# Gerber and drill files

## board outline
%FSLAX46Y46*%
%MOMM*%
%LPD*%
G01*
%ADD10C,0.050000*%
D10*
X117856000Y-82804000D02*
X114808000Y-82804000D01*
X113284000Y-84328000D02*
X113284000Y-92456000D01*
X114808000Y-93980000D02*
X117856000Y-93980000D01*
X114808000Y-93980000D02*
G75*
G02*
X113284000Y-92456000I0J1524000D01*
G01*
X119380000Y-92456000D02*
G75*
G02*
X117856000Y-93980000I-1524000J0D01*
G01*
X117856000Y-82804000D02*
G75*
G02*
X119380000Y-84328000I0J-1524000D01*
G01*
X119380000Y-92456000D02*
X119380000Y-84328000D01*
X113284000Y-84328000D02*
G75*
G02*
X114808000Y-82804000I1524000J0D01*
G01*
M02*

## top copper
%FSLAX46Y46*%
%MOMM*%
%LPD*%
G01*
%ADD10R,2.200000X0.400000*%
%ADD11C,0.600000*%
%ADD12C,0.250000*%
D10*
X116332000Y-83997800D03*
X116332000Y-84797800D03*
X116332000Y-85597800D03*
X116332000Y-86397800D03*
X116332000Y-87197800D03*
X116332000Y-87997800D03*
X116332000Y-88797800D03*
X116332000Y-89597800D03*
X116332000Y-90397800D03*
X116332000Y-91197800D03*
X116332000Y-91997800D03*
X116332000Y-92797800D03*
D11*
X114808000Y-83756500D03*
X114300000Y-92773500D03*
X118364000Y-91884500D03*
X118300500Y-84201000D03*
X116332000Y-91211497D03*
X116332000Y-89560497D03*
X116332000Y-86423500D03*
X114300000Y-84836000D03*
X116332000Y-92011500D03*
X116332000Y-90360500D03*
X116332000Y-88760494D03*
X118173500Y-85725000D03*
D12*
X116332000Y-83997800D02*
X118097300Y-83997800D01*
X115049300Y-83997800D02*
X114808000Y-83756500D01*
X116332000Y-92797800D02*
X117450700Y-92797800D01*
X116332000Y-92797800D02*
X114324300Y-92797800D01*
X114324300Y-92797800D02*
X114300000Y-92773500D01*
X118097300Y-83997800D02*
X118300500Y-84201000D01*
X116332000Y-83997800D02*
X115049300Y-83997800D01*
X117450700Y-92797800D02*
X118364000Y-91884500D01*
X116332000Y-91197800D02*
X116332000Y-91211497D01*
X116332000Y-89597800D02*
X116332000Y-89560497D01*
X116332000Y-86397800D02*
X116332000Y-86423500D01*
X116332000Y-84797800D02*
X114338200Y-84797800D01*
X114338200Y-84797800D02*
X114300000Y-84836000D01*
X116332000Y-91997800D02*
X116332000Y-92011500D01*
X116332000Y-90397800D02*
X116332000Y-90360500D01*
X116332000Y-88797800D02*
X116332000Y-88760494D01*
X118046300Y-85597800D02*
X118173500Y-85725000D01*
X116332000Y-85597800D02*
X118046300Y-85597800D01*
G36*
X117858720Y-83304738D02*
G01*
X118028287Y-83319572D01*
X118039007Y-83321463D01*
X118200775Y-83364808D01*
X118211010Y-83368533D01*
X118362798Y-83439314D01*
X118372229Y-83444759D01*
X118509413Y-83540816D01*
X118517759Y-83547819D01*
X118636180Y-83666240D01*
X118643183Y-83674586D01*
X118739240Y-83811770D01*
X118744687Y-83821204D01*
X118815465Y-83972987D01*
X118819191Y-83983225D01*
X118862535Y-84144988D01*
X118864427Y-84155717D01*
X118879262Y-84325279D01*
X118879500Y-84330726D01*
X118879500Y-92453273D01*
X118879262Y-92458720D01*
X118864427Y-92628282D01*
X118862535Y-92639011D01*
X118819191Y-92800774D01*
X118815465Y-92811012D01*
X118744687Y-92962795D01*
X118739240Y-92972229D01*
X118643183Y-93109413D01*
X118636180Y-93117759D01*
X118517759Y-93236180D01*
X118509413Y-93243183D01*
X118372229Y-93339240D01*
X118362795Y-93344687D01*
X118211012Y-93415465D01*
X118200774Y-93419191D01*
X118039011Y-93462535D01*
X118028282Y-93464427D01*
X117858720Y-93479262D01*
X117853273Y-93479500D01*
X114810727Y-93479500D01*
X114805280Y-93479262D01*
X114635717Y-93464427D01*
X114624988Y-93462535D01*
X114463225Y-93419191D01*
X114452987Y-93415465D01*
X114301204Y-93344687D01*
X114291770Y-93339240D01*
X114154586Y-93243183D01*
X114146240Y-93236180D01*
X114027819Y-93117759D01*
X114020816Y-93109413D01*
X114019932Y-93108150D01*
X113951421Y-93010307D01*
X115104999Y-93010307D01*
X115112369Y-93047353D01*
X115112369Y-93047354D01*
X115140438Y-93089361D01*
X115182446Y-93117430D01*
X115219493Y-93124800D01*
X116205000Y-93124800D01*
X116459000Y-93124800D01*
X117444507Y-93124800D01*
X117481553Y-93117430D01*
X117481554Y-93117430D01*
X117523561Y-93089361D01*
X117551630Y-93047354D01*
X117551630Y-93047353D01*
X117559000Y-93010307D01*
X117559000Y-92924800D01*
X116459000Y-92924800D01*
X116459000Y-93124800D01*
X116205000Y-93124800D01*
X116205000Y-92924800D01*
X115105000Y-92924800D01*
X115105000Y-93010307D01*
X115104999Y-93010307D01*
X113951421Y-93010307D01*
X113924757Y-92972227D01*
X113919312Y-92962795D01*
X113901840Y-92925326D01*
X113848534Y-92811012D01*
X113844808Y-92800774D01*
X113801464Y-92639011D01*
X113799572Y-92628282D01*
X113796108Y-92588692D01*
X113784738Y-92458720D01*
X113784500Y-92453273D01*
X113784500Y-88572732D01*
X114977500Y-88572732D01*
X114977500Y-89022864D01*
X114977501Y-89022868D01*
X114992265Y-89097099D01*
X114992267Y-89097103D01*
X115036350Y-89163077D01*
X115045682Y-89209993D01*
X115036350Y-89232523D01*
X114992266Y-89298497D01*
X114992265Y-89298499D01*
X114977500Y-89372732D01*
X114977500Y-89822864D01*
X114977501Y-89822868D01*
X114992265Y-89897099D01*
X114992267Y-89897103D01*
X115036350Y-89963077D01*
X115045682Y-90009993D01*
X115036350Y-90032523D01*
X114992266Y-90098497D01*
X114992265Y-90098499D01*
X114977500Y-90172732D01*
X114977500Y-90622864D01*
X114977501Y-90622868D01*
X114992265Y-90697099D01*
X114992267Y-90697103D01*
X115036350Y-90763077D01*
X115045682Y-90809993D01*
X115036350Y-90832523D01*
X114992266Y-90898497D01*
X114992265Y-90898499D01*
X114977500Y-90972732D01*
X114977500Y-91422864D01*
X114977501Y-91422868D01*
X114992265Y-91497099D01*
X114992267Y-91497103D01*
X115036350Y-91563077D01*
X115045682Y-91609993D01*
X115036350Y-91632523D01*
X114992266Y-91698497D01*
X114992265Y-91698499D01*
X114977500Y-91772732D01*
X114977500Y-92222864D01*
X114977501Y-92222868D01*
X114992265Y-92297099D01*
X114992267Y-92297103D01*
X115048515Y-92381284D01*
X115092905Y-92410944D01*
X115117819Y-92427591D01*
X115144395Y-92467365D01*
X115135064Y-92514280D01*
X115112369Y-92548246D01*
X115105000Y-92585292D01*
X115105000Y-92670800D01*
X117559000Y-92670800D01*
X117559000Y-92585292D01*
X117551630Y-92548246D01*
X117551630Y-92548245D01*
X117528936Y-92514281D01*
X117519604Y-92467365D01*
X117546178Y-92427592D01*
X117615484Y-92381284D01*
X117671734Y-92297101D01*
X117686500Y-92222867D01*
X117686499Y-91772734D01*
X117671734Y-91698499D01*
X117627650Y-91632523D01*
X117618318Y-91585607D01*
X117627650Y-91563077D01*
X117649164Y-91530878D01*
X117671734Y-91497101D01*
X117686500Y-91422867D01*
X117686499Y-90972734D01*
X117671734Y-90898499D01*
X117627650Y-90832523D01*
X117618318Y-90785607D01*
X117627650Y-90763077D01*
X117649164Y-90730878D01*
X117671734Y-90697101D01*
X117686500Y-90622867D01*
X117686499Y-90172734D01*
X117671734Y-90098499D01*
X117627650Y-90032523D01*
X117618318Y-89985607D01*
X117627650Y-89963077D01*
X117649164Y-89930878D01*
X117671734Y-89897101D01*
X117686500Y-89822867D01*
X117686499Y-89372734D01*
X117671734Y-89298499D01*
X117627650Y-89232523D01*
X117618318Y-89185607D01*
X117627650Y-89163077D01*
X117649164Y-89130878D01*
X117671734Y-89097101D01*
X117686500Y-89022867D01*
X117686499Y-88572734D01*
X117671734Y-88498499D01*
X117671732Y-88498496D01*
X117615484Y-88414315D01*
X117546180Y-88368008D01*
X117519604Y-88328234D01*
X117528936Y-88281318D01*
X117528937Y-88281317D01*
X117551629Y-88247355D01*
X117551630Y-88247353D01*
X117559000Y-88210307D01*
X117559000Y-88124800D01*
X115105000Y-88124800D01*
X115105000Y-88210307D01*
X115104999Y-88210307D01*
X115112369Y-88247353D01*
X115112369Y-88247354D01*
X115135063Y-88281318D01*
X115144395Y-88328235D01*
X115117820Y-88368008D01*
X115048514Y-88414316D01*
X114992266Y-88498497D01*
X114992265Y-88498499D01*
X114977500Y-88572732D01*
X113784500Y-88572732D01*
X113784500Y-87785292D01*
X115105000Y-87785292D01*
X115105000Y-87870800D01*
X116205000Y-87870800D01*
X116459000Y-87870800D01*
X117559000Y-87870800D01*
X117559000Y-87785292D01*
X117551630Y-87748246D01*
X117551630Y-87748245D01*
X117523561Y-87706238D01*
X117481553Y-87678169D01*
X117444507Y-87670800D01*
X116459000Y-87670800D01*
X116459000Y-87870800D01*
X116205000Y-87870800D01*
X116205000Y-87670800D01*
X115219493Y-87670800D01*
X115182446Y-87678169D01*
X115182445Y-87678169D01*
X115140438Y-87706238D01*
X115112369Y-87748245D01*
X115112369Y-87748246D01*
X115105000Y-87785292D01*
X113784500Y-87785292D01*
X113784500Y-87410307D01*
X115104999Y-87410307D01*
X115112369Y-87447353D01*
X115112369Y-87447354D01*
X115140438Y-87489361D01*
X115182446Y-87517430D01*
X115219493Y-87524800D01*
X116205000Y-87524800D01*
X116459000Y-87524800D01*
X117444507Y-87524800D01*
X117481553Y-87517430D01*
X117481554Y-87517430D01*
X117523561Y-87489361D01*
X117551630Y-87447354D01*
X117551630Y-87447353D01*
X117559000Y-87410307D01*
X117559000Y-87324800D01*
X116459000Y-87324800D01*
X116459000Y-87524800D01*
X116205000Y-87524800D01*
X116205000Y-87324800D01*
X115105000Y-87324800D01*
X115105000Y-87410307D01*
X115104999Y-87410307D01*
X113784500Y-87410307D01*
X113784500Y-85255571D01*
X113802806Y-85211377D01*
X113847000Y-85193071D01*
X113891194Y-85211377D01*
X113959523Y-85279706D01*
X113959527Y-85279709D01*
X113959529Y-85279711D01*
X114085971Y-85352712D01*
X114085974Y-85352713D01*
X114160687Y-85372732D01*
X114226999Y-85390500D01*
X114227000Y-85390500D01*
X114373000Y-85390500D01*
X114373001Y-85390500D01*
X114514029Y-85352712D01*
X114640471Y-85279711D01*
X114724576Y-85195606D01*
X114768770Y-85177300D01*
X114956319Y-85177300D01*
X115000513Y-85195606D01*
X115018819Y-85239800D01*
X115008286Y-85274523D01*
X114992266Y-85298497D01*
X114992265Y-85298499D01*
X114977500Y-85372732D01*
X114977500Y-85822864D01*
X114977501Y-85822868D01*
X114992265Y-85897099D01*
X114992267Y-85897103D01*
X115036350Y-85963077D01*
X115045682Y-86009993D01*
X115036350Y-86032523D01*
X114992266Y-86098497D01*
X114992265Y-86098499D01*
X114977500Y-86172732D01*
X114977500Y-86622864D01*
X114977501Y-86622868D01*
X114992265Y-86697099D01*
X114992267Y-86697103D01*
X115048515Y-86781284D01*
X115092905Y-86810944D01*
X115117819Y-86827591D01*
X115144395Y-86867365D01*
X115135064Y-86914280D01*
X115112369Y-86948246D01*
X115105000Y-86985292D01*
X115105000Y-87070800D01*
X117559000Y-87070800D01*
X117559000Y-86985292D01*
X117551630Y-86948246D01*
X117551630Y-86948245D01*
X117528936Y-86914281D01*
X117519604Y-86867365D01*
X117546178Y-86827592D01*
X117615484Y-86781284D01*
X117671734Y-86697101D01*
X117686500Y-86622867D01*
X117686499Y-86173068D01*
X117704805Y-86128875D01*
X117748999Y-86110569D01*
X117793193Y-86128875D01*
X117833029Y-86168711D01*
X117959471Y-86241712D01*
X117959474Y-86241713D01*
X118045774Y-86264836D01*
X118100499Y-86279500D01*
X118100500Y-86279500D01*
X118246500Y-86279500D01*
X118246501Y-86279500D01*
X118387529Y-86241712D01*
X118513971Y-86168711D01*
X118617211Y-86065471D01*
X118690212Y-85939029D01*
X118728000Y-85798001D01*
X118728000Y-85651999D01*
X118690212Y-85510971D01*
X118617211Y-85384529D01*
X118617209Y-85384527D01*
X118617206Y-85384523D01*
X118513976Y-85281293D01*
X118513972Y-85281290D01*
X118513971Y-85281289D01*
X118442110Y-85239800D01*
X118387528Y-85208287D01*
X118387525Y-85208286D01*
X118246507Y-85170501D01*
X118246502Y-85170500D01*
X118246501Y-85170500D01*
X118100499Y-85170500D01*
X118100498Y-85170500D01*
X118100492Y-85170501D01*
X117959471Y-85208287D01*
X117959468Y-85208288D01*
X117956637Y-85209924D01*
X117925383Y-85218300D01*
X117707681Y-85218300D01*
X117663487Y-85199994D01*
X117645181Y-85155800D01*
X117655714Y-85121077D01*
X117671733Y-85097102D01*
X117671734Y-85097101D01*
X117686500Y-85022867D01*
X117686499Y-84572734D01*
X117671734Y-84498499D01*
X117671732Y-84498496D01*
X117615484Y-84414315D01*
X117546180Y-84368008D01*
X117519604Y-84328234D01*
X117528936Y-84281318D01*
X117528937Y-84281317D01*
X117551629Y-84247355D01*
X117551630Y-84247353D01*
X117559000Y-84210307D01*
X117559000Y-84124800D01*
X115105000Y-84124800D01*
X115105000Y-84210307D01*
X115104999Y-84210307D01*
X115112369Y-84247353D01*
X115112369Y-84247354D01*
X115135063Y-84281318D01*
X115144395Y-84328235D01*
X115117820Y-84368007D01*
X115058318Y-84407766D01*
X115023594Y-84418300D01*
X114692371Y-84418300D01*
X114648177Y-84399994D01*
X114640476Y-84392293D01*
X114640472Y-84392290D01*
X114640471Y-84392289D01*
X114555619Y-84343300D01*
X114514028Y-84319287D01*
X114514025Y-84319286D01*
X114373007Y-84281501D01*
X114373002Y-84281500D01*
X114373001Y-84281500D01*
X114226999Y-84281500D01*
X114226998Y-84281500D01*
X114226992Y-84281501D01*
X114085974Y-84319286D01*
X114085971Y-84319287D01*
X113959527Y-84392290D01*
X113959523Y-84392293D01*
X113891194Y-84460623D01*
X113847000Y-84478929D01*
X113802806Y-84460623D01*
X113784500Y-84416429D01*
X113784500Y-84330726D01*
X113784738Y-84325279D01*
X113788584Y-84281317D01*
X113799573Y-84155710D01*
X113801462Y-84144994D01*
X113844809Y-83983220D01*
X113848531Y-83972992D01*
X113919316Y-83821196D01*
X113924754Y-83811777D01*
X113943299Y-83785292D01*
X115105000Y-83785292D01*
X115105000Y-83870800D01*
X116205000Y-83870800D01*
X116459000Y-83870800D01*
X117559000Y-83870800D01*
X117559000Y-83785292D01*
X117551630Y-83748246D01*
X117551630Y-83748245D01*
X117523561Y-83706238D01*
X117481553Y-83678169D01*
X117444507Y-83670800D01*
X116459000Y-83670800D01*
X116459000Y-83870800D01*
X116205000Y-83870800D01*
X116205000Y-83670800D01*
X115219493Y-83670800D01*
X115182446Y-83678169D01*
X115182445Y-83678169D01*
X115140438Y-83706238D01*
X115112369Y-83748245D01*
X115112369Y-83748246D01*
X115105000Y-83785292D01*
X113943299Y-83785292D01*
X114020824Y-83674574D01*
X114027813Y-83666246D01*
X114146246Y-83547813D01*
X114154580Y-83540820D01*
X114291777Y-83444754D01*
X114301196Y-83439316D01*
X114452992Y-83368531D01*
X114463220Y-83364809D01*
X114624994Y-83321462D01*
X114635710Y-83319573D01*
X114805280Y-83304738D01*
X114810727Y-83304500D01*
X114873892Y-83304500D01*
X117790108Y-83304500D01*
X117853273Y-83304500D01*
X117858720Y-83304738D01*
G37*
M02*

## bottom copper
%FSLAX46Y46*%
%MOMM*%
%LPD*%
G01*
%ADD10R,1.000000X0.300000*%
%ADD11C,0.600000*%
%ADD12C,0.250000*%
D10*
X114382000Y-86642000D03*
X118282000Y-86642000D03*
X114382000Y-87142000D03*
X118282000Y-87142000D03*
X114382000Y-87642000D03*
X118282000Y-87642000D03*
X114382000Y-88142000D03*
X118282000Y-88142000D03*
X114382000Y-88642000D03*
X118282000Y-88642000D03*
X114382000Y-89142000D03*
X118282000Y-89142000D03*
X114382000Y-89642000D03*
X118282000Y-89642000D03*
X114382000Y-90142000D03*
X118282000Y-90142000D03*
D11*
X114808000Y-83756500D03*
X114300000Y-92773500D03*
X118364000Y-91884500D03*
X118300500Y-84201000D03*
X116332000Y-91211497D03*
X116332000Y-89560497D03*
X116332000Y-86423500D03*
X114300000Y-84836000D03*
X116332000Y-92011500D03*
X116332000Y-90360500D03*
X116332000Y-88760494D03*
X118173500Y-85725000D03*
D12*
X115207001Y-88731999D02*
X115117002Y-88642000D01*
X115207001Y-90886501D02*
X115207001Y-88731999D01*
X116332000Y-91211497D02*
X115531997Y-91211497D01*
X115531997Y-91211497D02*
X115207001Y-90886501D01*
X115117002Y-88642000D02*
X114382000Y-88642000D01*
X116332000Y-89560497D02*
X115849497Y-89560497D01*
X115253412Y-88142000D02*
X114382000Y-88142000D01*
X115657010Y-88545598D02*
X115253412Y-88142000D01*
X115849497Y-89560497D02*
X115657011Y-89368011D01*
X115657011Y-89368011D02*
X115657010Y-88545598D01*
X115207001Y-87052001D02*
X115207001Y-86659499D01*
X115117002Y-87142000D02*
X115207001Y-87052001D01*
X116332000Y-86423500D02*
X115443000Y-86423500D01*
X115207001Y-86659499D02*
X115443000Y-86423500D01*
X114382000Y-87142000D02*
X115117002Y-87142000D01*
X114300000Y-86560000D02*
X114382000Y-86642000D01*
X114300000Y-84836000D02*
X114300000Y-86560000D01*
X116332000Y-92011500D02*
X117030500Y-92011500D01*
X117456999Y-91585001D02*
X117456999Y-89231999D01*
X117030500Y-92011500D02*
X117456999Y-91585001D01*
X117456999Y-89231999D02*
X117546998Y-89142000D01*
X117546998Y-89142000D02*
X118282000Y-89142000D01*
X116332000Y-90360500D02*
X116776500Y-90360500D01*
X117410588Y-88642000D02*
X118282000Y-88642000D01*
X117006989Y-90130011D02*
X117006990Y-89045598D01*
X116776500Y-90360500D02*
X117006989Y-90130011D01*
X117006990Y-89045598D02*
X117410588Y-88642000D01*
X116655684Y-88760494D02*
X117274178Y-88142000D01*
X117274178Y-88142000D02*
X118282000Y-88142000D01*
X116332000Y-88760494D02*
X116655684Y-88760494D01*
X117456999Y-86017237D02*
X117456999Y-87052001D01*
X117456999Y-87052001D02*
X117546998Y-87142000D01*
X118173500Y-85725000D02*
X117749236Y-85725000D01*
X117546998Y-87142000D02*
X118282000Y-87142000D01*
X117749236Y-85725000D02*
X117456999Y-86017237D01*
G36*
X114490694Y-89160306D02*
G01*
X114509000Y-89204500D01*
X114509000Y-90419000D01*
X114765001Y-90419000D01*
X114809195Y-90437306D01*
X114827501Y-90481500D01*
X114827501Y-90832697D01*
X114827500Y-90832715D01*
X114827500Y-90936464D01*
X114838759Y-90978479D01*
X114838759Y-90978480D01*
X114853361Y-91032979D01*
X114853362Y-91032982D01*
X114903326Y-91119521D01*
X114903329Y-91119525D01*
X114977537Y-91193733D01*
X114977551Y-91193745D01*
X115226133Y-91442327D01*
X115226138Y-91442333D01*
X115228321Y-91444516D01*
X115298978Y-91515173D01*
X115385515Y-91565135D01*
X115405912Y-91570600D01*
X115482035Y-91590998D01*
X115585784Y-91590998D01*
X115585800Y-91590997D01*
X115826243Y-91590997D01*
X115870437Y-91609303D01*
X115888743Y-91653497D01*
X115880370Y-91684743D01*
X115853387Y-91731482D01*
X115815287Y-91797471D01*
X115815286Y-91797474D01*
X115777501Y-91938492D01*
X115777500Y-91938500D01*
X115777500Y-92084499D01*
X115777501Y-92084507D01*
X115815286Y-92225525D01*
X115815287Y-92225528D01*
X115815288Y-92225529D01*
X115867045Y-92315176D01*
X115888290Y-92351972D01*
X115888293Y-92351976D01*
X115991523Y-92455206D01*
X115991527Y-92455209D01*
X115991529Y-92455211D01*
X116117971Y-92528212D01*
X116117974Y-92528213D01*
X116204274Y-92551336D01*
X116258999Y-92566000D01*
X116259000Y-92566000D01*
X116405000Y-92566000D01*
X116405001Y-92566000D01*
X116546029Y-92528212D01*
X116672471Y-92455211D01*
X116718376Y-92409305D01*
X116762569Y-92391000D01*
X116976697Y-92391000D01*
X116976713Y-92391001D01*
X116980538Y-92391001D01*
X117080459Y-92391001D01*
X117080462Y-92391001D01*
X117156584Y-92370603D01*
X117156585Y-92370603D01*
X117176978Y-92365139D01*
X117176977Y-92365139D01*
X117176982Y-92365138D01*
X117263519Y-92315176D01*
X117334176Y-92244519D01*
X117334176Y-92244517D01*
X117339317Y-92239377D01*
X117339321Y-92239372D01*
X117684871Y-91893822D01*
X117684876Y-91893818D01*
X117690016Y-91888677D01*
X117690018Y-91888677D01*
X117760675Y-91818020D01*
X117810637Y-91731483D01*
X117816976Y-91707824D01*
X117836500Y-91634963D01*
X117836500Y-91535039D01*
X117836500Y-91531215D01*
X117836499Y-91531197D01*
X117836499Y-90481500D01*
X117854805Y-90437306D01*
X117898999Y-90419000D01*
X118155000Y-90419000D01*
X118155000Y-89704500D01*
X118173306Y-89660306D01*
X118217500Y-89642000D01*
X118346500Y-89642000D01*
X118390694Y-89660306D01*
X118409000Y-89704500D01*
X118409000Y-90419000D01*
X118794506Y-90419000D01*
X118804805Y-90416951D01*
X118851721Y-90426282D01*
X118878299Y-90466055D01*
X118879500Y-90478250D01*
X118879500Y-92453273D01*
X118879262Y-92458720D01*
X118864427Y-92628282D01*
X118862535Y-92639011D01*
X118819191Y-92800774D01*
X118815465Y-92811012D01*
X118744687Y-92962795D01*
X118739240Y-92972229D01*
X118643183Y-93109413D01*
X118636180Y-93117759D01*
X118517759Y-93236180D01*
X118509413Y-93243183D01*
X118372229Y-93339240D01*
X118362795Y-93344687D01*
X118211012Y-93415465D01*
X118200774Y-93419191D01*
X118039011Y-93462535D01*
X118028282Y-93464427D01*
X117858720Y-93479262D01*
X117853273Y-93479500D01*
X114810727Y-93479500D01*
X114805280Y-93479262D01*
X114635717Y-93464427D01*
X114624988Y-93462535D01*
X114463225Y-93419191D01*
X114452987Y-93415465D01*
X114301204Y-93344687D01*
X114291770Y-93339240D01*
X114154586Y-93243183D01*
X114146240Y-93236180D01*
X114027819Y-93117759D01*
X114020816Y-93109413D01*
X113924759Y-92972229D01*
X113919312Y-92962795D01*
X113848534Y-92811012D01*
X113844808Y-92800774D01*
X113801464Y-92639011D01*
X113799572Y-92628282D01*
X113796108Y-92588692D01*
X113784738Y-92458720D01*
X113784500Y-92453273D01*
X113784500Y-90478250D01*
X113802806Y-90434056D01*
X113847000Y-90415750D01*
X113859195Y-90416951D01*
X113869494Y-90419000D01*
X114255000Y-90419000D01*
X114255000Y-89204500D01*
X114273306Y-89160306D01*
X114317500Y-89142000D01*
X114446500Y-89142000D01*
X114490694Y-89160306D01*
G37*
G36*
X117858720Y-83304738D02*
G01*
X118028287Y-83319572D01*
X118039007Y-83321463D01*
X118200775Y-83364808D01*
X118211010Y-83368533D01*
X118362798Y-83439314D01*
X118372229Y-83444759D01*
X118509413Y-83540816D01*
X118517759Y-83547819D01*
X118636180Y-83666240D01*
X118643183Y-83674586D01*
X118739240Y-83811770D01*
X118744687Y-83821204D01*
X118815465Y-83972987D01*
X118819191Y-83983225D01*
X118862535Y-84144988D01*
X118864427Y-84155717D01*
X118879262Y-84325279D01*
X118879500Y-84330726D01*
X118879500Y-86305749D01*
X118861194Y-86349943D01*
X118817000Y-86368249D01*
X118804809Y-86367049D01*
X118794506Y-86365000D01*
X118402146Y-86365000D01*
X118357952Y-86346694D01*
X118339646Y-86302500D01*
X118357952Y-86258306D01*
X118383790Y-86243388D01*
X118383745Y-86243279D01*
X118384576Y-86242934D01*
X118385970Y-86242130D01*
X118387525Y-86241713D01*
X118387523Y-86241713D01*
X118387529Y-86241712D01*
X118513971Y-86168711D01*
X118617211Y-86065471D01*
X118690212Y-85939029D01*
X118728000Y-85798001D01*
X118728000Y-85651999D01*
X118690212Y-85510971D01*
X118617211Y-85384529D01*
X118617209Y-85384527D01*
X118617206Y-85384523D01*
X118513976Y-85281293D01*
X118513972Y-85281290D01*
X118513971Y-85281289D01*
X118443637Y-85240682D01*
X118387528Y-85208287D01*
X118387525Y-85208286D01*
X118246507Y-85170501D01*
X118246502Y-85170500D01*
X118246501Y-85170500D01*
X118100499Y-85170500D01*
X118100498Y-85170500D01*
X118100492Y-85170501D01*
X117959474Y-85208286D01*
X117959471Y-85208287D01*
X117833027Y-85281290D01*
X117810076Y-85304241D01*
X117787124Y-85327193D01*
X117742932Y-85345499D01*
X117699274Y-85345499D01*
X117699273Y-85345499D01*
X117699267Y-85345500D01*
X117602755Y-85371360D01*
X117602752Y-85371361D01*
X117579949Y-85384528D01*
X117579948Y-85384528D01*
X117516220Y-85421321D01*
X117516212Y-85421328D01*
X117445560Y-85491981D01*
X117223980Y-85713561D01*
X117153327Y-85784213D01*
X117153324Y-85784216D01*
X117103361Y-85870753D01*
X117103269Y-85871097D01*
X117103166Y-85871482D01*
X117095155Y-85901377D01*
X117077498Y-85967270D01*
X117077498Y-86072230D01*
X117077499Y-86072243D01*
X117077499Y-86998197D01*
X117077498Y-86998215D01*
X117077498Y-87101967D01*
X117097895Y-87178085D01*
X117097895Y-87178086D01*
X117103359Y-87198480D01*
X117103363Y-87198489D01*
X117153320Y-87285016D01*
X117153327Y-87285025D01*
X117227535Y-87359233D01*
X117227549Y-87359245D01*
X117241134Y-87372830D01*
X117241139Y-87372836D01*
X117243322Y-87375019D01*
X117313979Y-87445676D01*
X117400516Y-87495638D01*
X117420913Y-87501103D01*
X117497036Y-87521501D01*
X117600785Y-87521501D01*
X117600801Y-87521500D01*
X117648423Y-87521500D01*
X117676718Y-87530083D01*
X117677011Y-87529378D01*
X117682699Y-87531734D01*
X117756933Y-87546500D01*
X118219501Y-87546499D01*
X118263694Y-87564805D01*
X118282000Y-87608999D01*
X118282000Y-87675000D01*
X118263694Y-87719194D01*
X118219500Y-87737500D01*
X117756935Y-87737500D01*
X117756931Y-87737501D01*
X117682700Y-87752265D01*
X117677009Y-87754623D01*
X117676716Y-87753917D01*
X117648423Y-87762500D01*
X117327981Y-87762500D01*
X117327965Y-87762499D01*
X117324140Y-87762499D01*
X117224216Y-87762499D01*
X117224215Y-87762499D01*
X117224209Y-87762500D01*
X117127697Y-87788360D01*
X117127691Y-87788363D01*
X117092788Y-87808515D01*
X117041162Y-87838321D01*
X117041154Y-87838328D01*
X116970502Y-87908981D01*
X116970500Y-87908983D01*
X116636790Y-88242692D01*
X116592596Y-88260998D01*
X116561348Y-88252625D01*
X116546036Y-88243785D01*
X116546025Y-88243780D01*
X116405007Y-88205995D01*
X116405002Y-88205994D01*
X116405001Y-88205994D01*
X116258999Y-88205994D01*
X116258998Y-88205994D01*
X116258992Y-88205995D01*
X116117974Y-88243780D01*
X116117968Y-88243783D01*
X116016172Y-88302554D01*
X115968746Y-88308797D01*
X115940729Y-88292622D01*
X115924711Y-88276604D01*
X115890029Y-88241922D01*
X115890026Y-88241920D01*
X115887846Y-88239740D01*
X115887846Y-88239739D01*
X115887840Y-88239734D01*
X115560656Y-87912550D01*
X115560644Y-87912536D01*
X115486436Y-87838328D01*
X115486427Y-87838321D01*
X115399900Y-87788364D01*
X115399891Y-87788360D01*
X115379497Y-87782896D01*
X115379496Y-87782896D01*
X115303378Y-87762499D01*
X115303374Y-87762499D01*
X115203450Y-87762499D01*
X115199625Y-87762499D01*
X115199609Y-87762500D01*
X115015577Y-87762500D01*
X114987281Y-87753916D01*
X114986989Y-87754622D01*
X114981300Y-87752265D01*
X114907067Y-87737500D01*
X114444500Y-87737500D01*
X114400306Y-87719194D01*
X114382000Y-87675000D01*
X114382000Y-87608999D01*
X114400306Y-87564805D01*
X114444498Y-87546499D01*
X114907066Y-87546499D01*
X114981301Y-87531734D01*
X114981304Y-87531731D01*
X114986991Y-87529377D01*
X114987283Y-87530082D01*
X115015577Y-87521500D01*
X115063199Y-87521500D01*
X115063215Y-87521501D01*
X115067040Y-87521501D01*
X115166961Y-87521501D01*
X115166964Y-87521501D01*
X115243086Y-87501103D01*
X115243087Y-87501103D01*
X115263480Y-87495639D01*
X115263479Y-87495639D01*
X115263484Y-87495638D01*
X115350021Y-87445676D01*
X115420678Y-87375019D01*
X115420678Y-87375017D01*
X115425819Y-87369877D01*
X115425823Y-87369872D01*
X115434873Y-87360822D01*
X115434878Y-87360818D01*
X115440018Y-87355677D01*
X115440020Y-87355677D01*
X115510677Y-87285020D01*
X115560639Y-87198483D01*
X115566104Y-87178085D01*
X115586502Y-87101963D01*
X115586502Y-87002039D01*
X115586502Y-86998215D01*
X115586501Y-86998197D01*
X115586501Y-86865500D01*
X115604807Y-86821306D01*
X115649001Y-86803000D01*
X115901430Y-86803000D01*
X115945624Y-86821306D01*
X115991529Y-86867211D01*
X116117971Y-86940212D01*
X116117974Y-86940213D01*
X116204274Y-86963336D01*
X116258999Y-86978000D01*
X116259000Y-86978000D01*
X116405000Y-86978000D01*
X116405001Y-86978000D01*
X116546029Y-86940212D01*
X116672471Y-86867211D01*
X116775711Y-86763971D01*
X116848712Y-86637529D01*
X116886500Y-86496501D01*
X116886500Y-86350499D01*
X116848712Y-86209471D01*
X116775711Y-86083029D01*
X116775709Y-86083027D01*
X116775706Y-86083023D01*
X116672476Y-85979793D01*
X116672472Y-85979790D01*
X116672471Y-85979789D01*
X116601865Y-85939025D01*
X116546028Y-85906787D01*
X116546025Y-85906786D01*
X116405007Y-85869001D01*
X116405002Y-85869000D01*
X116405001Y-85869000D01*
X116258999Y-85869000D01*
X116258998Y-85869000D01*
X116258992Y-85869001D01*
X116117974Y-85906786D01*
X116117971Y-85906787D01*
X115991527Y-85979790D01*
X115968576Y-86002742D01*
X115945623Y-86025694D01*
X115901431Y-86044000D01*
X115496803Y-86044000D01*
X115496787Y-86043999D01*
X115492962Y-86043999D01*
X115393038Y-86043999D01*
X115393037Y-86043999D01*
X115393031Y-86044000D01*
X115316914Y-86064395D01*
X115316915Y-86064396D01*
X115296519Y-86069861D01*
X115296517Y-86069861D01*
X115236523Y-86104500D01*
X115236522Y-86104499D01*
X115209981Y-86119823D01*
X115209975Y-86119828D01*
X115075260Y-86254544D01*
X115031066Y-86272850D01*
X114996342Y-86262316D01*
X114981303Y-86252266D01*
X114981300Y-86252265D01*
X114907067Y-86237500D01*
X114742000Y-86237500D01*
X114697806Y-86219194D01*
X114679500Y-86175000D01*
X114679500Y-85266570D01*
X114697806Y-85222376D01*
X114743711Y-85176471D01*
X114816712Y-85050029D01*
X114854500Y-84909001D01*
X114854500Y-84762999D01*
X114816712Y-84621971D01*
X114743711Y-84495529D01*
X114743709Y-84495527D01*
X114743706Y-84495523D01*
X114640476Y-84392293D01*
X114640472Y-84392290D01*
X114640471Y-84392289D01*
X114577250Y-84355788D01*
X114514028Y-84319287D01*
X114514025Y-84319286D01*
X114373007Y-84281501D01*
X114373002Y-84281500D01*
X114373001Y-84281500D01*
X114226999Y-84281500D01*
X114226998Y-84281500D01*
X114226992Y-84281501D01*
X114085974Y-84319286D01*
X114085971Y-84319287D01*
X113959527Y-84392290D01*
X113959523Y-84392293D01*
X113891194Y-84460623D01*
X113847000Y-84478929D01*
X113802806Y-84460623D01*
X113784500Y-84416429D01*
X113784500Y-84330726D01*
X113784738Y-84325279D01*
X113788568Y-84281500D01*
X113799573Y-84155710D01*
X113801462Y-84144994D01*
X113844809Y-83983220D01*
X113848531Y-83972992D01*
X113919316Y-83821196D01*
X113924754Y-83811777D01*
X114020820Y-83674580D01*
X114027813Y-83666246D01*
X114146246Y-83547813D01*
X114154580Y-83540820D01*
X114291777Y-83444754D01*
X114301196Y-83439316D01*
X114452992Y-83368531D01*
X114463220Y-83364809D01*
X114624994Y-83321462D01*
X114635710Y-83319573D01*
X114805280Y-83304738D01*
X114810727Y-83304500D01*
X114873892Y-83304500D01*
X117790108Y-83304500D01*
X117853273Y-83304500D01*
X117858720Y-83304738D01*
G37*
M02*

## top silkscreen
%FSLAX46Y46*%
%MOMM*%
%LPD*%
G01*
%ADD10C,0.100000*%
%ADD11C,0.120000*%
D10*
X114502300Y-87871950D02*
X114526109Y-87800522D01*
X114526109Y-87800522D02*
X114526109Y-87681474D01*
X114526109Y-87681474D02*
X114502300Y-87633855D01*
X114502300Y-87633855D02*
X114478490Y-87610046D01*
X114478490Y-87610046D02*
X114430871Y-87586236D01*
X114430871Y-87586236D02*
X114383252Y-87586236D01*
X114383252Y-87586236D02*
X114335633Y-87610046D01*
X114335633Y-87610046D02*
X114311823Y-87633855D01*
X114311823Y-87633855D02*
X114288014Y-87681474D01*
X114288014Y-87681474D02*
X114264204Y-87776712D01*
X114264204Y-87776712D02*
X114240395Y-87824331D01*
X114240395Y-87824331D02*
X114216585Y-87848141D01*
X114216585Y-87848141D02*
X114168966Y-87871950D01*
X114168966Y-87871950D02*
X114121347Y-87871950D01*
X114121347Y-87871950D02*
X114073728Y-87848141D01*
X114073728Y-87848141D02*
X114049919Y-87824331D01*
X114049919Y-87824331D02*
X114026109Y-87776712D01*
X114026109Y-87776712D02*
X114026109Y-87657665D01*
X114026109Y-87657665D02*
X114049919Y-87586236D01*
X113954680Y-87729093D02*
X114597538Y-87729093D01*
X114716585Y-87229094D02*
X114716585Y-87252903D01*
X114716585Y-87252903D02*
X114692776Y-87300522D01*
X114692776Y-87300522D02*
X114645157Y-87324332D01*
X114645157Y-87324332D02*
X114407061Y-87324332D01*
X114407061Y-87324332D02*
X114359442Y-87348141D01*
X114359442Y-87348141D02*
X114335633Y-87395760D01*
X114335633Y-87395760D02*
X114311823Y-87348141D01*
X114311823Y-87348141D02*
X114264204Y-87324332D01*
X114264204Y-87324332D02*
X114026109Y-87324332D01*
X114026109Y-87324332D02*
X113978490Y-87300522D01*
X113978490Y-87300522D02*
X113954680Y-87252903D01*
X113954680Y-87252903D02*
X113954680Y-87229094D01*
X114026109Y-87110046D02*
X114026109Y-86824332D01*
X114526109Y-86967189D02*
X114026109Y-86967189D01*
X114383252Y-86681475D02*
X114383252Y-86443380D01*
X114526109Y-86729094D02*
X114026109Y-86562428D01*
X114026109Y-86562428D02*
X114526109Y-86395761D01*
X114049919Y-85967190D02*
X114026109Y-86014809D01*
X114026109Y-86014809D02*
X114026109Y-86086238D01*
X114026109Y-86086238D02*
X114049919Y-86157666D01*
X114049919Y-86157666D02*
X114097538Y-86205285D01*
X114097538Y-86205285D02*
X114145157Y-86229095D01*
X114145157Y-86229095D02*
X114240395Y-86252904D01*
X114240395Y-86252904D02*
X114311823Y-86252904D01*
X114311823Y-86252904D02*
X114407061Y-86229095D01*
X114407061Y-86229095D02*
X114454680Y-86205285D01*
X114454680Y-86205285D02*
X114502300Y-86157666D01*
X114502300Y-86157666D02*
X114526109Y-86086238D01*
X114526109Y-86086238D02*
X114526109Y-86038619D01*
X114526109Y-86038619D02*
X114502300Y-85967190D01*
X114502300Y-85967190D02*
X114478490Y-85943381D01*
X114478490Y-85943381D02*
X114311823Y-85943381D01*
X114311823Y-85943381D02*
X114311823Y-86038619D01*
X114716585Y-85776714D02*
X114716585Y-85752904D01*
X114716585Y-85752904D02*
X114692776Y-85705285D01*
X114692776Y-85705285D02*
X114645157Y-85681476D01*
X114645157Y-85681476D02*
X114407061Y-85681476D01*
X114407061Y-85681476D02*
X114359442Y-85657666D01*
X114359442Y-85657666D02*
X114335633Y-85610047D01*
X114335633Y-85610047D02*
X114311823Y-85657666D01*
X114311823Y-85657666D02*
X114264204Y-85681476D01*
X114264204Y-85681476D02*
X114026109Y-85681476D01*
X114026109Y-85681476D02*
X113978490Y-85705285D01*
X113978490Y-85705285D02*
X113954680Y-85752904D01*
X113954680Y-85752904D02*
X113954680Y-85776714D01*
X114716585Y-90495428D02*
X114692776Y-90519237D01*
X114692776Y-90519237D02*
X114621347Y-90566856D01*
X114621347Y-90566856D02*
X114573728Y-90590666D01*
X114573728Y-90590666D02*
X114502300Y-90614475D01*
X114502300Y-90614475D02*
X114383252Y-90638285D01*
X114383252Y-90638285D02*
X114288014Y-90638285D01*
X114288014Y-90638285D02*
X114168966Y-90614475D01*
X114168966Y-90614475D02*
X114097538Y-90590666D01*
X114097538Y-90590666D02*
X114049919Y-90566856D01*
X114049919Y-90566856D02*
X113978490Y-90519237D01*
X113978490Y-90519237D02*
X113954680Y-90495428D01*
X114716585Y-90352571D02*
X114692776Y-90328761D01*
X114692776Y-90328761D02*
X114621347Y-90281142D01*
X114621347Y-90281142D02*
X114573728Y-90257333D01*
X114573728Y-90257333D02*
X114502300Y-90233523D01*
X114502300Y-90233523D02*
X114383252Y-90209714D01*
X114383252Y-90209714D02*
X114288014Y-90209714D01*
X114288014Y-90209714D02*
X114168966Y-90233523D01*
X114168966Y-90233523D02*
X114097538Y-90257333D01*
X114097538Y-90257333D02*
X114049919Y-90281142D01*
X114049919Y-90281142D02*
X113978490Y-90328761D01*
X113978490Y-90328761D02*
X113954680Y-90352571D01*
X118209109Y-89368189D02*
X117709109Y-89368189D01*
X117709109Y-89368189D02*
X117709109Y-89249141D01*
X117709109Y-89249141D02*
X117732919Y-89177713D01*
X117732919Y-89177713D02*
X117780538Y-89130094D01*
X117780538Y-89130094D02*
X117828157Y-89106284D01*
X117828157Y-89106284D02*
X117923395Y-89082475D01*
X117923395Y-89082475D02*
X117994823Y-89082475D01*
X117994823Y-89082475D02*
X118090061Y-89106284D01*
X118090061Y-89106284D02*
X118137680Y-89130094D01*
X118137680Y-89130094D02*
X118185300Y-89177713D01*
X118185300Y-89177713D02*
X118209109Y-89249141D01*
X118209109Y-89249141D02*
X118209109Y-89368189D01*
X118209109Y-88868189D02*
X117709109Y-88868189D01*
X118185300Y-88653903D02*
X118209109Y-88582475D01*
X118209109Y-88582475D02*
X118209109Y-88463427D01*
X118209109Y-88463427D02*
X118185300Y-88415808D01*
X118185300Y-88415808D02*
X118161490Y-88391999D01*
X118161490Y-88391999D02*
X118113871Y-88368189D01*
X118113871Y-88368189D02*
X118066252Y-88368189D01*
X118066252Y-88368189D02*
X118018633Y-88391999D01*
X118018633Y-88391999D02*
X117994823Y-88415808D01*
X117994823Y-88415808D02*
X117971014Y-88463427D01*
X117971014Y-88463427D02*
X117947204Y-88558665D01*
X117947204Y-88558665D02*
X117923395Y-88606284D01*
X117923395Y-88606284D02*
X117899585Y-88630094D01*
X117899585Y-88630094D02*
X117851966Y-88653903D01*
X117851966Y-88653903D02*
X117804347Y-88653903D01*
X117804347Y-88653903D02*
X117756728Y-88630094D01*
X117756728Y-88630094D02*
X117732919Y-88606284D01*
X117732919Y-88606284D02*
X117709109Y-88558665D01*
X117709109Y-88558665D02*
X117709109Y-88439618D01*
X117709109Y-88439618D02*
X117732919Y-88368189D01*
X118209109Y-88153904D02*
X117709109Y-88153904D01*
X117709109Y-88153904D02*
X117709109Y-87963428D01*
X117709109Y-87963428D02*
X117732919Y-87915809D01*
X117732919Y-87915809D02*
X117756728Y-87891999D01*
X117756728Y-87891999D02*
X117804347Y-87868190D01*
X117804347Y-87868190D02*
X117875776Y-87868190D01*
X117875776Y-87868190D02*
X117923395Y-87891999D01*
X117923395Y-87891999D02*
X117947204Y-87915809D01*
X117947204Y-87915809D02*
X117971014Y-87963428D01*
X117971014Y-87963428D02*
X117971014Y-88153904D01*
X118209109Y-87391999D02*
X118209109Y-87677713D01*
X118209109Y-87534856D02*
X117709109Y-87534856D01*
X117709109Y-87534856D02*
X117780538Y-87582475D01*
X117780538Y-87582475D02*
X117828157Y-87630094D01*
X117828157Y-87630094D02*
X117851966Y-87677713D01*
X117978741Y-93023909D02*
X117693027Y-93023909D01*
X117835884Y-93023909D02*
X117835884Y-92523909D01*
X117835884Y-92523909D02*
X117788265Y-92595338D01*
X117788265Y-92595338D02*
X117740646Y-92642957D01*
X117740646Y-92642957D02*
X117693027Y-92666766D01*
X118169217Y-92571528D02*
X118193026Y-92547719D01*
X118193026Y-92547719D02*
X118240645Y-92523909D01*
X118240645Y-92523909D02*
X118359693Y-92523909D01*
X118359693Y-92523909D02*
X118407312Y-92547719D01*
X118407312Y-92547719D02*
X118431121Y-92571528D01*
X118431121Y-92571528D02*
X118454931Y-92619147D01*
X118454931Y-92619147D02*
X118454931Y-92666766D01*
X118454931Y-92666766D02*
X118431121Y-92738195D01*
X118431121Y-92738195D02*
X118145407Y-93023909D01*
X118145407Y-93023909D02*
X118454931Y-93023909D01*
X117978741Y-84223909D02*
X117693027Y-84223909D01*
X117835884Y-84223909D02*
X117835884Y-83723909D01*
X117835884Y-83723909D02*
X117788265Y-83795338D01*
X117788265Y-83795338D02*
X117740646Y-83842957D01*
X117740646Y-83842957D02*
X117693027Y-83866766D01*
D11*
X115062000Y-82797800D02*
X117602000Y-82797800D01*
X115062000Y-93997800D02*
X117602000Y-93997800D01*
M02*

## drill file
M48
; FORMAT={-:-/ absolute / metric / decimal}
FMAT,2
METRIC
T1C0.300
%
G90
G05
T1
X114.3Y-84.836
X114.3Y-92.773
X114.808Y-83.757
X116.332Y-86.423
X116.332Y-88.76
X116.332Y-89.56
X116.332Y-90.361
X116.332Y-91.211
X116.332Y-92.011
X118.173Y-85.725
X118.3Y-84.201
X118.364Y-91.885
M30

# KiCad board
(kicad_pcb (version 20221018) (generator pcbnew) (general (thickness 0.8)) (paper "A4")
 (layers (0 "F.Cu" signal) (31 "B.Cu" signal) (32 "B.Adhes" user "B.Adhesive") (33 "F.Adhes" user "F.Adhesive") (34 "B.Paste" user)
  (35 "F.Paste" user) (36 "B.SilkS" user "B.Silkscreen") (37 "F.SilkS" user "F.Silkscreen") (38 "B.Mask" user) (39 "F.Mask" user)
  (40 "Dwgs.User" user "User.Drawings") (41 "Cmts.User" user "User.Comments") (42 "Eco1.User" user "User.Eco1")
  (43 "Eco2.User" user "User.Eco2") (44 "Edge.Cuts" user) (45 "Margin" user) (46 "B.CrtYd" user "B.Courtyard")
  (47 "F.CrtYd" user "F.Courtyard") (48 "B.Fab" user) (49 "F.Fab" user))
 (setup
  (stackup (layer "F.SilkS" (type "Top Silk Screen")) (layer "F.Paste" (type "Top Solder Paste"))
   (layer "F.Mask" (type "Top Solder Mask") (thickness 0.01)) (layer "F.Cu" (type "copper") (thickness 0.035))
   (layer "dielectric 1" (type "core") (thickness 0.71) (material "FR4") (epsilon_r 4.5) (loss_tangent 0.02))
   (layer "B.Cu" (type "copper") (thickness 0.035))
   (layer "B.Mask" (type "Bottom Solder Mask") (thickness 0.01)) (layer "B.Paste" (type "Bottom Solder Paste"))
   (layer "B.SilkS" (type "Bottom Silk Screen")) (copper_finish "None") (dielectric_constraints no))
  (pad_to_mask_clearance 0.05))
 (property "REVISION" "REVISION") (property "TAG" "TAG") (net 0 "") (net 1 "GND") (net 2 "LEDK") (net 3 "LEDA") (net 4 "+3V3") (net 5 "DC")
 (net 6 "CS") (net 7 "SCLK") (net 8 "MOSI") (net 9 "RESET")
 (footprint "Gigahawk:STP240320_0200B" (layer "F.Cu") (at 116.332 83.9978)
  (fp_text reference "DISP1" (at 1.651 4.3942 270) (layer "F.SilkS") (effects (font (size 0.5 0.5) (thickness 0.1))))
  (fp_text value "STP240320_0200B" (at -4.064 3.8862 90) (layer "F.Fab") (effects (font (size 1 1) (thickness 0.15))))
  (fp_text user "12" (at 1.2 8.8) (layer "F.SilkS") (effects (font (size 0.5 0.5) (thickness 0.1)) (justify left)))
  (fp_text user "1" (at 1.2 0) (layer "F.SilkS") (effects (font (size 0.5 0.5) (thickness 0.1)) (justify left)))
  (fp_line (start -1.27 -1.2) (end 1.27 -1.2) (stroke (width 0.12) (type solid)) (layer "F.SilkS"))
  (fp_line (start -1.27 10) (end 1.27 10) (stroke (width 0.12) (type solid)) (layer "F.SilkS"))
  (pad "1" smd rect (at 0 0 90) (size 0.4 2.2) (layers "F.Cu" "F.Paste" "F.Mask") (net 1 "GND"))
  (pad "2" smd rect (at 0 0.8 90) (size 0.4 2.2) (layers "F.Cu" "F.Paste" "F.Mask") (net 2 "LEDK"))
  (pad "3" smd rect (at 0 1.6 90) (size 0.4 2.2) (layers "F.Cu" "F.Paste" "F.Mask") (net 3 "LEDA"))
  (pad "4" smd rect (at 0 2.4 90) (size 0.4 2.2) (layers "F.Cu" "F.Paste" "F.Mask") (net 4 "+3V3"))
  (pad "5" smd rect (at 0 3.2 90) (size 0.4 2.2) (layers "F.Cu" "F.Paste" "F.Mask") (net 1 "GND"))
  (pad "6" smd rect (at 0 4 90) (size 0.4 2.2) (layers "F.Cu" "F.Paste" "F.Mask") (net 1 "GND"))
  (pad "7" smd rect (at 0 4.8 90) (size 0.4 2.2) (layers "F.Cu" "F.Paste" "F.Mask") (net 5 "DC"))
  (pad "8" smd rect (at 0 5.6 90) (size 0.4 2.2) (layers "F.Cu" "F.Paste" "F.Mask") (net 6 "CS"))
  (pad "9" smd rect (at 0 6.4 90) (size 0.4 2.2) (layers "F.Cu" "F.Paste" "F.Mask") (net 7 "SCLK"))
  (pad "10" smd rect (at 0 7.2 90) (size 0.4 2.2) (layers "F.Cu" "F.Paste" "F.Mask") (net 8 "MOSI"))
  (pad "11" smd rect (at 0 8 90) (size 0.4 2.2) (layers "F.Cu" "F.Paste" "F.Mask") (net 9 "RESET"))
  (pad "12" smd rect (at 0 8.8 90) (size 0.4 2.2) (layers "F.Cu" "F.Paste" "F.Mask") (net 1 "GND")))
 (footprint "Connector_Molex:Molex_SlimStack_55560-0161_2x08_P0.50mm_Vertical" (layer "B.Cu") (at 116.332 88.392 -90)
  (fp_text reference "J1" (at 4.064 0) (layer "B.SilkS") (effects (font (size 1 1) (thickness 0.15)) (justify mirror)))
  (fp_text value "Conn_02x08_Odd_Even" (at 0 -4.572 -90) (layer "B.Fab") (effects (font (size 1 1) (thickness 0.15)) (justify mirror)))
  (pad "1" smd rect (at -1.75 1.95 270) (size 0.3 1) (layers "B.Cu" "B.Paste" "B.Mask") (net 2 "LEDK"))
  (pad "2" smd rect (at -1.75 -1.95 270) (size 0.3 1) (layers "B.Cu" "B.Paste" "B.Mask") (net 1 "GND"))
  (pad "3" smd rect (at -1.25 1.95 270) (size 0.3 1) (layers "B.Cu" "B.Paste" "B.Mask") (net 4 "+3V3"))
  (pad "4" smd rect (at -1.25 -1.95 270) (size 0.3 1) (layers "B.Cu" "B.Paste" "B.Mask") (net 3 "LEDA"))
  (pad "5" smd rect (at -0.75 1.95 270) (size 0.3 1) (layers "B.Cu" "B.Paste" "B.Mask") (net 1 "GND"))
  (pad "6" smd rect (at -0.75 -1.95 270) (size 0.3 1) (layers "B.Cu" "B.Paste" "B.Mask") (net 1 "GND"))
  (pad "7" smd rect (at -0.25 1.95 270) (size 0.3 1) (layers "B.Cu" "B.Paste" "B.Mask") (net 6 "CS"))
  (pad "8" smd rect (at -0.25 -1.95 270) (size 0.3 1) (layers "B.Cu" "B.Paste" "B.Mask") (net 5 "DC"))
  (pad "9" smd rect (at 0.25 1.95 270) (size 0.3 1) (layers "B.Cu" "B.Paste" "B.Mask") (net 8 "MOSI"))
  (pad "10" smd rect (at 0.25 -1.95 270) (size 0.3 1) (layers "B.Cu" "B.Paste" "B.Mask") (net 7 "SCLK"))
  (pad "11" smd rect (at 0.75 1.95 270) (size 0.3 1) (layers "B.Cu" "B.Paste" "B.Mask") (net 1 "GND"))
  (pad "12" smd rect (at 0.75 -1.95 270) (size 0.3 1) (layers "B.Cu" "B.Paste" "B.Mask") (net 9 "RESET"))
  (pad "13" smd rect (at 1.25 1.95 270) (size 0.3 1) (layers "B.Cu" "B.Paste" "B.Mask") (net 1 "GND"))
  (pad "14" smd rect (at 1.25 -1.95 270) (size 0.3 1) (layers "B.Cu" "B.Paste" "B.Mask") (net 1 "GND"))
  (pad "15" smd rect (at 1.75 1.95 270) (size 0.3 1) (layers "B.Cu" "B.Paste" "B.Mask") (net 1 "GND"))
  (pad "16" smd rect (at 1.75 -1.95 270) (size 0.3 1) (layers "B.Cu" "B.Paste" "B.Mask") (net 1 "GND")))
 (gr_line (start 117.856 82.804) (end 114.808 82.804) (stroke (width 0.05) (type solid)) (layer "Edge.Cuts"))
 (gr_line (start 113.284 84.328) (end 113.284 92.456) (stroke (width 0.05) (type solid)) (layer "Edge.Cuts"))
 (gr_line (start 114.808 93.98) (end 117.856 93.98) (stroke (width 0.05) (type solid)) (layer "Edge.Cuts"))
 (gr_arc (start 114.808 93.98) (mid 113.730369 93.533631) (end 113.284 92.456) (stroke (width 0.05) (type solid)) (layer "Edge.Cuts"))
 (gr_arc (start 119.38 92.456) (mid 118.933631 93.533631) (end 117.856 93.98) (stroke (width 0.05) (type solid)) (layer "Edge.Cuts"))
 (gr_arc (start 117.856 82.804) (mid 118.933631 83.250369) (end 119.38 84.328) (stroke (width 0.05) (type solid)) (layer "Edge.Cuts"))
 (gr_line (start 119.38 92.456) (end 119.38 84.328) (stroke (width 0.05) (type solid)) (layer "Edge.Cuts"))
 (gr_arc (start 113.284 84.328) (mid 113.730369 83.250369) (end 114.808 82.804) (stroke (width 0.05) (type solid)) (layer "Edge.Cuts"))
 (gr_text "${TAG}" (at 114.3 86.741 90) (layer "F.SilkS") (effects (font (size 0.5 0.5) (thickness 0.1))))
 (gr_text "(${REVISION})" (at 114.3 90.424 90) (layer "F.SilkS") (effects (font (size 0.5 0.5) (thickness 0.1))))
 (segment (start 116.332 83.9978) (end 118.0973 83.9978) (width 0.25) (layer "F.Cu") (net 1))
 (segment (start 115.0493 83.9978) (end 114.808 83.7565) (width 0.25) (layer "F.Cu") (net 1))
 (segment (start 116.332 92.7978) (end 117.4507 92.7978) (width 0.25) (layer "F.Cu") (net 1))
 (segment (start 116.332 92.7978) (end 114.3243 92.7978) (width 0.25) (layer "F.Cu") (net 1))
 (segment (start 114.3243 92.7978) (end 114.3 92.7735) (width 0.25) (layer "F.Cu") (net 1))
 (segment (start 118.0973 83.9978) (end 118.3005 84.201) (width 0.25) (layer "F.Cu") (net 1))
 (segment (start 116.332 83.9978) (end 115.0493 83.9978) (width 0.25) (layer "F.Cu") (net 1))
 (segment (start 117.4507 92.7978) (end 118.364 91.8845) (width 0.25) (layer "F.Cu") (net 1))
 (via (at 114.808 83.7565) (size 0.6) (drill 0.3) (layers "F.Cu" "B.Cu") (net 1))
 (via (at 114.3 92.7735) (size 0.6) (drill 0.3) (layers "F.Cu" "B.Cu") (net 1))
 (via (at 118.364 91.8845) (size 0.6) (drill 0.3) (layers "F.Cu" "B.Cu") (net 1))
 (via (at 118.3005 84.201) (size 0.6) (drill 0.3) (layers "F.Cu" "B.Cu") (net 1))
 (segment (start 116.332 91.1978) (end 116.332 91.211497) (width 0.25) (layer "F.Cu") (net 8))
 (via (at 116.332 91.211497) (size 0.6) (drill 0.3) (layers "F.Cu" "B.Cu") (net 8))
 (segment (start 115.207001 88.731999) (end 115.117002 88.642) (width 0.25) (layer "B.Cu") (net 8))
 (segment (start 115.207001 90.886501) (end 115.207001 88.731999) (width 0.25) (layer "B.Cu") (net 8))
 (segment (start 116.332 91.211497) (end 115.531997 91.211497) (width 0.25) (layer "B.Cu") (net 8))
 (segment (start 115.531997 91.211497) (end 115.207001 90.886501) (width 0.25) (layer "B.Cu") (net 8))
 (segment (start 115.117002 88.642) (end 114.382 88.642) (width 0.25) (layer "B.Cu") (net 8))
 (segment (start 116.332 89.5978) (end 116.332 89.560497) (width 0.25) (layer "F.Cu") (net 6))
 (via (at 116.332 89.560497) (size 0.6) (drill 0.3) (layers "F.Cu" "B.Cu") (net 6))
 (segment (start 116.332 89.560497) (end 115.849497 89.560497) (width 0.25) (layer "B.Cu") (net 6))
 (segment (start 115.253412 88.142) (end 114.382 88.142) (width 0.25) (layer "B.Cu") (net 6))
 (segment (start 115.65701 88.545598) (end 115.253412 88.142) (width 0.25) (layer "B.Cu") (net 6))
 (segment (start 115.849497 89.560497) (end 115.657011 89.368011) (width 0.25) (layer "B.Cu") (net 6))
 (segment (start 115.657011 89.368011) (end 115.65701 88.545598) (width 0.25) (layer "B.Cu") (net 6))
 (segment (start 116.332 86.3978) (end 116.332 86.4235) (width 0.25) (layer "F.Cu") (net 4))
 (via (at 116.332 86.4235) (size 0.6) (drill 0.3) (layers "F.Cu" "B.Cu") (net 4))
 (segment (start 115.207001 87.052001) (end 115.207001 86.659499) (width 0.25) (layer "B.Cu") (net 4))
 (segment (start 115.117002 87.142) (end 115.207001 87.052001) (width 0.25) (layer "B.Cu") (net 4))
 (segment (start 116.332 86.4235) (end 115.443 86.4235) (width 0.25) (layer "B.Cu") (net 4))
 (segment (start 115.207001 86.659499) (end 115.443 86.4235) (width 0.25) (layer "B.Cu") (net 4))
 (segment (start 114.382 87.142) (end 115.117002 87.142) (width 0.25) (layer "B.Cu") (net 4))
 (segment (start 116.332 84.7978) (end 114.3382 84.7978) (width 0.25) (layer "F.Cu") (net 2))
 (segment (start 114.3382 84.7978) (end 114.3 84.836) (width 0.25) (layer "F.Cu") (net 2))
 (via (at 114.3 84.836) (size 0.6) (drill 0.3) (layers "F.Cu" "B.Cu") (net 2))
 (segment (start 114.3 86.56) (end 114.382 86.642) (width 0.25) (layer "B.Cu") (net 2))
 (segment (start 114.3 84.836) (end 114.3 86.56) (width 0.25) (layer "B.Cu") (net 2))
 (segment (start 116.332 91.9978) (end 116.332 92.0115) (width 0.25) (layer "F.Cu") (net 9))
 (via (at 116.332 92.0115) (size 0.6) (drill 0.3) (layers "F.Cu" "B.Cu") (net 9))
 (segment (start 116.332 92.0115) (end 117.0305 92.0115) (width 0.25) (layer "B.Cu") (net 9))
 (segment (start 117.456999 91.585001) (end 117.456999 89.231999) (width 0.25) (layer "B.Cu") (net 9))
 (segment (start 117.0305 92.0115) (end 117.456999 91.585001) (width 0.25) (layer "B.Cu") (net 9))
 (segment (start 117.456999 89.231999) (end 117.546998 89.142) (width 0.25) (layer "B.Cu") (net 9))
 (segment (start 117.546998 89.142) (end 118.282 89.142) (width 0.25) (layer "B.Cu") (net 9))
 (segment (start 116.332 90.3978) (end 116.332 90.3605) (width 0.25) (layer "F.Cu") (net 7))
 (via (at 116.332 90.3605) (size 0.6) (drill 0.3) (layers "F.Cu" "B.Cu") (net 7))
 (segment (start 116.332 90.3605) (end 116.7765 90.3605) (width 0.25) (layer "B.Cu") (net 7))
 (segment (start 117.410588 88.642) (end 118.282 88.642) (width 0.25) (layer "B.Cu") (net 7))
 (segment (start 117.006989 90.130011) (end 117.00699 89.045598) (width 0.25) (layer "B.Cu") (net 7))
 (segment (start 116.7765 90.3605) (end 117.006989 90.130011) (width 0.25) (layer "B.Cu") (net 7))
 (segment (start 117.00699 89.045598) (end 117.410588 88.642) (width 0.25) (layer "B.Cu") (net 7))
 (segment (start 116.332 88.7978) (end 116.332 88.760494) (width 0.25) (layer "F.Cu") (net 5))
 (via (at 116.332 88.760494) (size 0.6) (drill 0.3) (layers "F.Cu" "B.Cu") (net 5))
 (segment (start 116.655684 88.760494) (end 117.274178 88.142) (width 0.25) (layer "B.Cu") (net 5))
 (segment (start 117.274178 88.142) (end 118.282 88.142) (width 0.25) (layer "B.Cu") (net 5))
 (segment (start 116.332 88.760494) (end 116.655684 88.760494) (width 0.25) (layer "B.Cu") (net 5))
 (segment (start 118.0463 85.5978) (end 118.1735 85.725) (width 0.25) (layer "F.Cu") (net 3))
 (segment (start 116.332 85.5978) (end 118.0463 85.5978) (width 0.25) (layer "F.Cu") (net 3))
 (via (at 118.1735 85.725) (size 0.6) (drill 0.3) (layers "F.Cu" "B.Cu") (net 3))
 (segment (start 117.456999 86.017237) (end 117.456999 87.052001) (width 0.25) (layer "B.Cu") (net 3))
 (segment (start 117.456999 87.052001) (end 117.546998 87.142) (width 0.25) (layer "B.Cu") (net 3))
 (segment (start 118.1735 85.725) (end 117.749236 85.725) (width 0.25) (layer "B.Cu") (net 3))
 (segment (start 117.546998 87.142) (end 118.282 87.142) (width 0.25) (layer "B.Cu") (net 3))
 (segment (start 117.749236 85.725) (end 117.456999 86.017237) (width 0.25) (layer "B.Cu") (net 3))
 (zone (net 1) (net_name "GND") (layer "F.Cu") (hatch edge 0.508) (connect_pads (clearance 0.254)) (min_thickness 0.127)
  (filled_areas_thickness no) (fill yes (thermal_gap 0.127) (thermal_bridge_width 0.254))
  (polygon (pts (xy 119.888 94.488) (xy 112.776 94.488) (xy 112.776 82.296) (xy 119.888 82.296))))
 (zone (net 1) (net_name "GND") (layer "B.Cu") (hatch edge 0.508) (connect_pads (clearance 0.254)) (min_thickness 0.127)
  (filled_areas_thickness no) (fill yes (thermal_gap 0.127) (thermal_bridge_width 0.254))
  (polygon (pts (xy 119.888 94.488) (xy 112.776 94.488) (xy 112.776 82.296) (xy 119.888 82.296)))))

